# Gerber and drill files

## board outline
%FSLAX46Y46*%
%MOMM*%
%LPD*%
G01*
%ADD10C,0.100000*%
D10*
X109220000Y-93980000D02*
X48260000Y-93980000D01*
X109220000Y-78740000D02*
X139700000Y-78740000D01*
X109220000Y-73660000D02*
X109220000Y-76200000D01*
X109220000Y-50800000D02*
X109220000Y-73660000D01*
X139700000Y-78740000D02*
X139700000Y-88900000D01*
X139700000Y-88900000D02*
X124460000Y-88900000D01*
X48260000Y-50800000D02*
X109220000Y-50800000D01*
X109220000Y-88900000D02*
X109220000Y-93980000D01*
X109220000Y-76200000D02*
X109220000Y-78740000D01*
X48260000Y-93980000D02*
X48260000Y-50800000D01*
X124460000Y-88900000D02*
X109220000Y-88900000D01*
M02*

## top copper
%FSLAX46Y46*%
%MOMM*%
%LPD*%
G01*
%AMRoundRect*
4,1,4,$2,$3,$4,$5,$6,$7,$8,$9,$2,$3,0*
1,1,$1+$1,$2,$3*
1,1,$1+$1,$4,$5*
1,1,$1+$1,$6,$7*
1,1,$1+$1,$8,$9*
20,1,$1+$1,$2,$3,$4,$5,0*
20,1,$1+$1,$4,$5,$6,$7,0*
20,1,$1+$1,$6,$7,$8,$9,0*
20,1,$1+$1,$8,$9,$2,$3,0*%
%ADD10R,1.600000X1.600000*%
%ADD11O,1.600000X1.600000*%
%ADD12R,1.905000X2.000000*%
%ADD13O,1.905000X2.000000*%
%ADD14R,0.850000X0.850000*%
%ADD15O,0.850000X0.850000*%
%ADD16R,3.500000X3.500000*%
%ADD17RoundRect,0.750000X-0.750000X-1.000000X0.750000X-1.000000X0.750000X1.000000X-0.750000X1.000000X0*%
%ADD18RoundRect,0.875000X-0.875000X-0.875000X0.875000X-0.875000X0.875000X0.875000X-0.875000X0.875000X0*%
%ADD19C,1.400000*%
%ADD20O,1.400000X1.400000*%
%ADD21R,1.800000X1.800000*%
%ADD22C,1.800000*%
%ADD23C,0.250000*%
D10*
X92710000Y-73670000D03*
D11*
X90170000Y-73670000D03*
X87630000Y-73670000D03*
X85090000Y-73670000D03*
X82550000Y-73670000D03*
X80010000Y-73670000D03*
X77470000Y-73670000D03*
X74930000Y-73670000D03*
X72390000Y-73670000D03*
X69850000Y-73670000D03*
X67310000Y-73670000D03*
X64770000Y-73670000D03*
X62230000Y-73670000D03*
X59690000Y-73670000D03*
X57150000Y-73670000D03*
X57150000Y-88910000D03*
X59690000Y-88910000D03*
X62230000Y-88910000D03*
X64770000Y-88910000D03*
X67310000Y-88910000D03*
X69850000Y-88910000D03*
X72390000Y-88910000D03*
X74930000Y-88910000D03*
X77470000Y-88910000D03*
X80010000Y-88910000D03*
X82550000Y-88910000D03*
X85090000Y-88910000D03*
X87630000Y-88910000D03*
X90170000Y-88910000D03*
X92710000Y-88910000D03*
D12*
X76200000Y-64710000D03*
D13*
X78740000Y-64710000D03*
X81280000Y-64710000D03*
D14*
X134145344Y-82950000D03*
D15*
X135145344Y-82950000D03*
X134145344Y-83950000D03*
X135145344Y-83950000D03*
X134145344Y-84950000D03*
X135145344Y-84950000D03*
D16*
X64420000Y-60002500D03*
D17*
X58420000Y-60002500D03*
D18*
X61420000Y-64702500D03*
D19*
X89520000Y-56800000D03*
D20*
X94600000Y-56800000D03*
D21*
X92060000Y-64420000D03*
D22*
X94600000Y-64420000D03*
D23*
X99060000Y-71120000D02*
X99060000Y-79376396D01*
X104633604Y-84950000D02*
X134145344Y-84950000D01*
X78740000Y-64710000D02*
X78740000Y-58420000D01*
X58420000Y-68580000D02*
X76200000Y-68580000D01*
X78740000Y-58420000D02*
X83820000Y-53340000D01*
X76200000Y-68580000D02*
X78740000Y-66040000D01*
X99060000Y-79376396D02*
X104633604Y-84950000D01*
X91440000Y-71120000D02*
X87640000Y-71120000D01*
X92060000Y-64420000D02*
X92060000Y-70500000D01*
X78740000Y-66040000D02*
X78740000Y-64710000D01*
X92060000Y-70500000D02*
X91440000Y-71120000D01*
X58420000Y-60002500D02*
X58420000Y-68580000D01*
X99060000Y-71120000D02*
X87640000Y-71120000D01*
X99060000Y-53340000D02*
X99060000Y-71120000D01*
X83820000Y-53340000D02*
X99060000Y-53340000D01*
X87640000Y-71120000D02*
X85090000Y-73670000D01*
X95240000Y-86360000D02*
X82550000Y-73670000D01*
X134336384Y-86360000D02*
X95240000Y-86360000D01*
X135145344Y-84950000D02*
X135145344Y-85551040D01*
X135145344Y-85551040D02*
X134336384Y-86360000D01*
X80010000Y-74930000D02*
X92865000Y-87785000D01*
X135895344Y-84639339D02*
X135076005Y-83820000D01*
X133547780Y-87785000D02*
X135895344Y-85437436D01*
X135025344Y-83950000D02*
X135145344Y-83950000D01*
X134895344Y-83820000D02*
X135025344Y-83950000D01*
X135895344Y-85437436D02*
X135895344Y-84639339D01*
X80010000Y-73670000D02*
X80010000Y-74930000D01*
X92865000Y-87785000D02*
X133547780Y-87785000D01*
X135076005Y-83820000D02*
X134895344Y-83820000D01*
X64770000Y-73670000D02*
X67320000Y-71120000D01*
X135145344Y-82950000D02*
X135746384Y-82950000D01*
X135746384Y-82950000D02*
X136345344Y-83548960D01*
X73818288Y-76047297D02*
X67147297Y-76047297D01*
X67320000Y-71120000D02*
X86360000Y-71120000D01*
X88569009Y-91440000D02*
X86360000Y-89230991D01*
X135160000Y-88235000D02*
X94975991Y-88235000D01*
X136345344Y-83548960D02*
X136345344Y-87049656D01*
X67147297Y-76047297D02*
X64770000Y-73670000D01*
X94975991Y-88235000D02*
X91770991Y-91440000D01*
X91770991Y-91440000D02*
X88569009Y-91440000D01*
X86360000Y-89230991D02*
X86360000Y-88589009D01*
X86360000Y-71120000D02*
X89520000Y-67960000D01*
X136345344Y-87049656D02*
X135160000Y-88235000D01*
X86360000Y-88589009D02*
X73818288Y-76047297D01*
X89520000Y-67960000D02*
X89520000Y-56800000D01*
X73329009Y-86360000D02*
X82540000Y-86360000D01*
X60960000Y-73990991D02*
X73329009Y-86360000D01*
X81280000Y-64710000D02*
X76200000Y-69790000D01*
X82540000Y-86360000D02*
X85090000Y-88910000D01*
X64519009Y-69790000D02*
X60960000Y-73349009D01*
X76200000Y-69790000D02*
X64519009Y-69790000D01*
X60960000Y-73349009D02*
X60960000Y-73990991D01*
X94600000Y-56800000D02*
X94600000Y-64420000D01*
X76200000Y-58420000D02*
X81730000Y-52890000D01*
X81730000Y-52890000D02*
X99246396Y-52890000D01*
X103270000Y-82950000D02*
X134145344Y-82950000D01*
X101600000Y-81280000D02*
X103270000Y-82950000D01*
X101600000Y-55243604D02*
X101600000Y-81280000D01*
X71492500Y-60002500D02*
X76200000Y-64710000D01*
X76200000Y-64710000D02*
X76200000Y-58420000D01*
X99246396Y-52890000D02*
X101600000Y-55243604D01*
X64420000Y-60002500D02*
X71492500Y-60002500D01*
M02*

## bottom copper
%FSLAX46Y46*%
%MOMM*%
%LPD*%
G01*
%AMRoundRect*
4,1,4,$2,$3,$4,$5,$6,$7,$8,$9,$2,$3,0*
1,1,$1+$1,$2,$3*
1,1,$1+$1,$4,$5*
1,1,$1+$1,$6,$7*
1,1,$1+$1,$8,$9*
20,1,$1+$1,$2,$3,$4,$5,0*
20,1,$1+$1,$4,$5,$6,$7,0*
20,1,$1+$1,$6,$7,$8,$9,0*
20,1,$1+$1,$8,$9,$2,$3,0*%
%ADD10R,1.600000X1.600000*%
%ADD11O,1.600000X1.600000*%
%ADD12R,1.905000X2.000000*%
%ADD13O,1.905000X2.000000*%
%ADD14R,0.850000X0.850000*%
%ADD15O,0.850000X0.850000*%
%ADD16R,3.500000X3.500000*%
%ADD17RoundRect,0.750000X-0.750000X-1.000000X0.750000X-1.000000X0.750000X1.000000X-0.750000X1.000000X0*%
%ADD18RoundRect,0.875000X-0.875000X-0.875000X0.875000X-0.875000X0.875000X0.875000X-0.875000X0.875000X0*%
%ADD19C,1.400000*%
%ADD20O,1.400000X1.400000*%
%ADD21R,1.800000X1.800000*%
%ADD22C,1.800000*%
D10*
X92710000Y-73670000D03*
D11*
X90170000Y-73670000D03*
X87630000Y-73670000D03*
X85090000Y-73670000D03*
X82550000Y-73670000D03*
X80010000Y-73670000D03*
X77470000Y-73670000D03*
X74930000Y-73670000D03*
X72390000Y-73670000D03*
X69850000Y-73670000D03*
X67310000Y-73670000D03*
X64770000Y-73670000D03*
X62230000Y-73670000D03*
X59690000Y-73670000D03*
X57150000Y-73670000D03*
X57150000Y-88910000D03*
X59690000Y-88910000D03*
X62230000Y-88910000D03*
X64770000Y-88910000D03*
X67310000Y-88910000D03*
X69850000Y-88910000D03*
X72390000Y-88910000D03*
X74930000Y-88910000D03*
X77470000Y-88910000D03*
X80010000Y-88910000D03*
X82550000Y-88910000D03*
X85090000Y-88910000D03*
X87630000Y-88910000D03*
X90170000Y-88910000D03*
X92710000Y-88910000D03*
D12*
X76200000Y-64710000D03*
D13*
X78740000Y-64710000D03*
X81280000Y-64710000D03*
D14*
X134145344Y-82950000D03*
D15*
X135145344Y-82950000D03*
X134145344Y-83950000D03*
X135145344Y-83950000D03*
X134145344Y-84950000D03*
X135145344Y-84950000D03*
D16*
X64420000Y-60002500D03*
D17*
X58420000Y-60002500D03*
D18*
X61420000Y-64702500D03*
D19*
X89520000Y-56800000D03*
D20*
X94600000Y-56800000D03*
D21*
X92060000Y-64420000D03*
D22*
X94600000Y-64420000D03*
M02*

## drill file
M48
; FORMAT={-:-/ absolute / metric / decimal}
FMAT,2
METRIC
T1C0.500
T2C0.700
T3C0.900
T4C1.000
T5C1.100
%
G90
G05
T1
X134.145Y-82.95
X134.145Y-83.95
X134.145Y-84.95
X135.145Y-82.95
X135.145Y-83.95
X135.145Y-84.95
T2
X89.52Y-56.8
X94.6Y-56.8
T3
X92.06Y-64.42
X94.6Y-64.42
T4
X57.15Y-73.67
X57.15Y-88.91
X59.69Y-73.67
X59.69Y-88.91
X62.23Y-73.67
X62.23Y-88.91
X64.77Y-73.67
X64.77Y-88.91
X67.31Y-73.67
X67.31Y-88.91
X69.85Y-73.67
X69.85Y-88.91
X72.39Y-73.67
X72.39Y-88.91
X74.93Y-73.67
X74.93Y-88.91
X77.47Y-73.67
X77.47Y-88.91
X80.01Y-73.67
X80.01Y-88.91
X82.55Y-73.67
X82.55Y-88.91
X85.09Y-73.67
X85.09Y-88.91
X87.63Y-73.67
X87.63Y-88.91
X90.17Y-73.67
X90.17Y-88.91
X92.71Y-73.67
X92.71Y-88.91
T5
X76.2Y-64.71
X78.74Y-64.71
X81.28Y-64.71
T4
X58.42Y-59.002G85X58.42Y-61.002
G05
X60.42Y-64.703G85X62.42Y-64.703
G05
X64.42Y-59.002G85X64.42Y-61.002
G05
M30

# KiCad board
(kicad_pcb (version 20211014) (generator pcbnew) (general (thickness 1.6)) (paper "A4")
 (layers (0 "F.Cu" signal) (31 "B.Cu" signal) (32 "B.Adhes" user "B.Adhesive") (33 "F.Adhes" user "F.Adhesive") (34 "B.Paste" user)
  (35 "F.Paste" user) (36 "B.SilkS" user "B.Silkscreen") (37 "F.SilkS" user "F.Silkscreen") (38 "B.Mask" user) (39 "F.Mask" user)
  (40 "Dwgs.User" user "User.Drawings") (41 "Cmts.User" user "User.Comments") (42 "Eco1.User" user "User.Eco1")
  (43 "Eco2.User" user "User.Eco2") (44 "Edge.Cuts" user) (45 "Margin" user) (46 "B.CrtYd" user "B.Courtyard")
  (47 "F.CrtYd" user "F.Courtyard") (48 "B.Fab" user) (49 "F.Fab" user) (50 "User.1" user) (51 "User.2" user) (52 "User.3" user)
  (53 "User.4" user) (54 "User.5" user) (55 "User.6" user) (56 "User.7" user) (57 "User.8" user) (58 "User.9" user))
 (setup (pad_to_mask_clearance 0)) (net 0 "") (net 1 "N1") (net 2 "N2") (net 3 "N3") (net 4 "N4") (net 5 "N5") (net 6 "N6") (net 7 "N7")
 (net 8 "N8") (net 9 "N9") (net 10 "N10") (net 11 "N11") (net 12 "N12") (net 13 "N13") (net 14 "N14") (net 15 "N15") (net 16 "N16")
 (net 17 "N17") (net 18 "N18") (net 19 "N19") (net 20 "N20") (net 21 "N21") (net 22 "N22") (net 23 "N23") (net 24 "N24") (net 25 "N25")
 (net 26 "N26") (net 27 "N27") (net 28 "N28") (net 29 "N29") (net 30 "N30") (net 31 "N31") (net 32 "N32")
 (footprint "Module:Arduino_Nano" (layer "F.Cu") (at 92.71 73.67 -90)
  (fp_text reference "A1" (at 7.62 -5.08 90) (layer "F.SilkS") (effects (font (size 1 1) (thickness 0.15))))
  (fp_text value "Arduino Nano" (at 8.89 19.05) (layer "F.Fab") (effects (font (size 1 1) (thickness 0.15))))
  (pad "1" thru_hole rect (at 0 0 270) (size 1.6 1.6) (drill 1) (layers *.Cu *.Mask) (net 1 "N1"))
  (pad "2" thru_hole oval (at 0 2.54 270) (size 1.6 1.6) (drill 1) (layers *.Cu *.Mask) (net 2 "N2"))
  (pad "3" thru_hole oval (at 0 5.08 270) (size 1.6 1.6) (drill 1) (layers *.Cu *.Mask) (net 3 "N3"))
  (pad "4" thru_hole oval (at 0 7.62 270) (size 1.6 1.6) (drill 1) (layers *.Cu *.Mask) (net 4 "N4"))
  (pad "5" thru_hole oval (at 0 10.16 270) (size 1.6 1.6) (drill 1) (layers *.Cu *.Mask) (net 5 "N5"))
  (pad "6" thru_hole oval (at 0 12.7 270) (size 1.6 1.6) (drill 1) (layers *.Cu *.Mask) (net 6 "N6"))
  (pad "7" thru_hole oval (at 0 15.24 270) (size 1.6 1.6) (drill 1) (layers *.Cu *.Mask) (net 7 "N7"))
  (pad "8" thru_hole oval (at 0 17.78 270) (size 1.6 1.6) (drill 1) (layers *.Cu *.Mask) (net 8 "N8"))
  (pad "9" thru_hole oval (at 0 20.32 270) (size 1.6 1.6) (drill 1) (layers *.Cu *.Mask) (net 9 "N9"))
  (pad "10" thru_hole oval (at 0 22.86 270) (size 1.6 1.6) (drill 1) (layers *.Cu *.Mask) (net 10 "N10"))
  (pad "11" thru_hole oval (at 0 25.4 270) (size 1.6 1.6) (drill 1) (layers *.Cu *.Mask) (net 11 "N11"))
  (pad "12" thru_hole oval (at 0 27.94 270) (size 1.6 1.6) (drill 1) (layers *.Cu *.Mask) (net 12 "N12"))
  (pad "13" thru_hole oval (at 0 30.48 270) (size 1.6 1.6) (drill 1) (layers *.Cu *.Mask) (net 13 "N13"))
  (pad "14" thru_hole oval (at 0 33.02 270) (size 1.6 1.6) (drill 1) (layers *.Cu *.Mask) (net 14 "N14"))
  (pad "15" thru_hole oval (at 0 35.56 270) (size 1.6 1.6) (drill 1) (layers *.Cu *.Mask) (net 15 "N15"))
  (pad "16" thru_hole oval (at 15.24 35.56 270) (size 1.6 1.6) (drill 1) (layers *.Cu *.Mask) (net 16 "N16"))
  (pad "17" thru_hole oval (at 15.24 33.02 270) (size 1.6 1.6) (drill 1) (layers *.Cu *.Mask) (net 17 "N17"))
  (pad "18" thru_hole oval (at 15.24 30.48 270) (size 1.6 1.6) (drill 1) (layers *.Cu *.Mask) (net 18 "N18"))
  (pad "19" thru_hole oval (at 15.24 27.94 270) (size 1.6 1.6) (drill 1) (layers *.Cu *.Mask) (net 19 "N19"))
  (pad "20" thru_hole oval (at 15.24 25.4 270) (size 1.6 1.6) (drill 1) (layers *.Cu *.Mask) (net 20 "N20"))
  (pad "21" thru_hole oval (at 15.24 22.86 270) (size 1.6 1.6) (drill 1) (layers *.Cu *.Mask) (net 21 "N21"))
  (pad "22" thru_hole oval (at 15.24 20.32 270) (size 1.6 1.6) (drill 1) (layers *.Cu *.Mask) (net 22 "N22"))
  (pad "23" thru_hole oval (at 15.24 17.78 270) (size 1.6 1.6) (drill 1) (layers *.Cu *.Mask) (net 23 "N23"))
  (pad "24" thru_hole oval (at 15.24 15.24 270) (size 1.6 1.6) (drill 1) (layers *.Cu *.Mask) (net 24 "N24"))
  (pad "25" thru_hole oval (at 15.24 12.7 270) (size 1.6 1.6) (drill 1) (layers *.Cu *.Mask) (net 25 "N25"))
  (pad "26" thru_hole oval (at 15.24 10.16 270) (size 1.6 1.6) (drill 1) (layers *.Cu *.Mask) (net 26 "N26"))
  (pad "27" thru_hole oval (at 15.24 7.62 270) (size 1.6 1.6) (drill 1) (layers *.Cu *.Mask) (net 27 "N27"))
  (pad "28" thru_hole oval (at 15.24 5.08 270) (size 1.6 1.6) (drill 1) (layers *.Cu *.Mask) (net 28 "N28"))
  (pad "29" thru_hole oval (at 15.24 2.54 270) (size 1.6 1.6) (drill 1) (layers *.Cu *.Mask) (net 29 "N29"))
  (pad "30" thru_hole oval (at 15.24 0 270) (size 1.6 1.6) (drill 1) (layers *.Cu *.Mask) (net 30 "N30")))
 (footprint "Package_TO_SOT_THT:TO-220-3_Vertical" (layer "F.Cu") (at 76.2 64.71)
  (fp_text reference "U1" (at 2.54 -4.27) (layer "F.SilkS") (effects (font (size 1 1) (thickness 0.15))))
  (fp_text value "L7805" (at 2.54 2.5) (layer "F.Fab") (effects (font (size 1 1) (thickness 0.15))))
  (pad "1" thru_hole rect (at 0 0) (size 1.905 2) (drill 1.1) (layers *.Cu *.Mask) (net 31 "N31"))
  (pad "2" thru_hole oval (at 2.54 0) (size 1.905 2) (drill 1.1) (layers *.Cu *.Mask) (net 4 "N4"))
  (pad "3" thru_hole oval (at 5.08 0) (size 1.905 2) (drill 1.1) (layers *.Cu *.Mask) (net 27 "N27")))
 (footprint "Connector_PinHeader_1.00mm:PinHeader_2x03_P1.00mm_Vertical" (layer "F.Cu") (at 134.145344 82.95)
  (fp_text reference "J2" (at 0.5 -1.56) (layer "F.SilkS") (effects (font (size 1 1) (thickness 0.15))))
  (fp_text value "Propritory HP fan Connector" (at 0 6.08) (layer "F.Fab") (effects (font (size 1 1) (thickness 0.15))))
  (pad "1" thru_hole rect (at 0 0) (size 0.85 0.85) (drill 0.5) (layers *.Cu *.Mask) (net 31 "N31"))
  (pad "2" thru_hole oval (at 1 0) (size 0.85 0.85) (drill 0.5) (layers *.Cu *.Mask) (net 12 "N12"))
  (pad "3" thru_hole oval (at 0 1) (size 0.85 0.85) (drill 0.5) (layers *.Cu *.Mask) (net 31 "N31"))
  (pad "4" thru_hole oval (at 1 1) (size 0.85 0.85) (drill 0.5) (layers *.Cu *.Mask) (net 6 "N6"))
  (pad "5" thru_hole oval (at 0 2) (size 0.85 0.85) (drill 0.5) (layers *.Cu *.Mask) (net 4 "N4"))
  (pad "6" thru_hole oval (at 1 2) (size 0.85 0.85) (drill 0.5) (layers *.Cu *.Mask) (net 5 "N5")))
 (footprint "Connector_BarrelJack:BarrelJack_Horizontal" (layer "F.Cu") (at 64.42 60.0025)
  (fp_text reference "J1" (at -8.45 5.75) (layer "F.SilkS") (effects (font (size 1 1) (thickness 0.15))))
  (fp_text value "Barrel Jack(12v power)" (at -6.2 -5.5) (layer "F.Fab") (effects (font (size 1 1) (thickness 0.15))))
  (pad "1" thru_hole rect (at 0 0) (size 3.5 3.5) (drill oval 1 3) (layers *.Cu *.Mask) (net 31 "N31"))
  (pad "2" thru_hole roundrect (at -6 0) (size 3 3.5) (drill oval 1 3) (layers *.Cu *.Mask) (roundrect_rratio 0.25) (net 4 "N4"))
  (pad "3" thru_hole roundrect (at -3 4.7) (size 3.5 3.5) (drill oval 3 1) (layers *.Cu *.Mask) (roundrect_rratio 0.25)))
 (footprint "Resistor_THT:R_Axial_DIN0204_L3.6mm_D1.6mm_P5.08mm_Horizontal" (layer "F.Cu") (at 89.52 56.8)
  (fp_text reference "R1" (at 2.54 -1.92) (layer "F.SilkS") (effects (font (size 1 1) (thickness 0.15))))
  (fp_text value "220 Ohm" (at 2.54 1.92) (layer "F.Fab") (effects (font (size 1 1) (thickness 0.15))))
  (pad "1" thru_hole circle (at 0 0) (size 1.4 1.4) (drill 0.7) (layers *.Cu *.Mask) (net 12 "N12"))
  (pad "2" thru_hole oval (at 5.08 0) (size 1.4 1.4) (drill 0.7) (layers *.Cu *.Mask) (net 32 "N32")))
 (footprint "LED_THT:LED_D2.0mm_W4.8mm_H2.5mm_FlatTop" (layer "F.Cu") (at 92.06 64.42)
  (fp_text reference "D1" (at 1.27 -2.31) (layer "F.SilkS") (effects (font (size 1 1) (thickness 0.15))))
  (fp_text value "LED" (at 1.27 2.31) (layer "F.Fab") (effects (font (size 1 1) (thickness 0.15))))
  (pad "1" thru_hole rect (at 0 0) (size 1.8 1.8) (drill 0.9) (layers *.Cu *.Mask) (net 4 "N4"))
  (pad "2" thru_hole circle (at 2.54 0) (size 1.8 1.8) (drill 0.9) (layers *.Cu *.Mask) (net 32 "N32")))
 (gr_line (start 109.22 93.98) (end 48.26 93.98) (layer "Edge.Cuts") (width 0.1))
 (gr_line (start 109.22 78.74) (end 139.7 78.74) (layer "Edge.Cuts") (width 0.1))
 (gr_line (start 109.22 73.66) (end 109.22 76.2) (layer "Edge.Cuts") (width 0.1))
 (gr_line (start 109.22 50.8) (end 109.22 73.66) (layer "Edge.Cuts") (width 0.1))
 (gr_line (start 139.7 78.74) (end 139.7 88.9) (layer "Edge.Cuts") (width 0.1))
 (gr_line (start 139.7 88.9) (end 124.46 88.9) (layer "Edge.Cuts") (width 0.1))
 (gr_line (start 48.26 50.8) (end 109.22 50.8) (layer "Edge.Cuts") (width 0.1))
 (gr_line (start 109.22 88.9) (end 109.22 93.98) (layer "Edge.Cuts") (width 0.1))
 (gr_line (start 109.22 76.2) (end 109.22 78.74) (layer "Edge.Cuts") (width 0.1))
 (gr_line (start 48.26 93.98) (end 48.26 50.8) (layer "Edge.Cuts") (width 0.1))
 (gr_line (start 124.46 88.9) (end 109.22 88.9) (layer "Edge.Cuts") (width 0.1))
 (segment (start 99.06 71.12) (end 99.06 79.376396) (width 0.25) (layer "F.Cu") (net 4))
 (segment (start 104.633604 84.95) (end 134.145344 84.95) (width 0.25) (layer "F.Cu") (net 4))
 (segment (start 78.74 64.71) (end 78.74 58.42) (width 0.25) (layer "F.Cu") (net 4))
 (segment (start 58.42 68.58) (end 76.2 68.58) (width 0.25) (layer "F.Cu") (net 4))
 (segment (start 78.74 58.42) (end 83.82 53.34) (width 0.25) (layer "F.Cu") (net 4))
 (segment (start 76.2 68.58) (end 78.74 66.04) (width 0.25) (layer "F.Cu") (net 4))
 (segment (start 99.06 79.376396) (end 104.633604 84.95) (width 0.25) (layer "F.Cu") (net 4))
 (segment (start 91.44 71.12) (end 87.64 71.12) (width 0.25) (layer "F.Cu") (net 4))
 (segment (start 92.06 64.42) (end 92.06 70.5) (width 0.25) (layer "F.Cu") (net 4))
 (segment (start 78.74 66.04) (end 78.74 64.71) (width 0.25) (layer "F.Cu") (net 4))
 (segment (start 92.06 70.5) (end 91.44 71.12) (width 0.25) (layer "F.Cu") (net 4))
 (segment (start 58.42 60.0025) (end 58.42 68.58) (width 0.25) (layer "F.Cu") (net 4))
 (segment (start 99.06 71.12) (end 87.64 71.12) (width 0.25) (layer "F.Cu") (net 4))
 (segment (start 99.06 53.34) (end 99.06 71.12) (width 0.25) (layer "F.Cu") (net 4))
 (segment (start 83.82 53.34) (end 99.06 53.34) (width 0.25) (layer "F.Cu") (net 4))
 (segment (start 87.64 71.12) (end 85.09 73.67) (width 0.25) (layer "F.Cu") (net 4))
 (segment (start 95.24 86.36) (end 82.55 73.67) (width 0.25) (layer "F.Cu") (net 5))
 (segment (start 134.336384 86.36) (end 95.24 86.36) (width 0.25) (layer "F.Cu") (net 5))
 (segment (start 135.145344 84.95) (end 135.145344 85.55104) (width 0.25) (layer "F.Cu") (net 5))
 (segment (start 135.145344 85.55104) (end 134.336384 86.36) (width 0.25) (layer "F.Cu") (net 5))
 (segment (start 80.01 74.93) (end 92.865 87.785) (width 0.25) (layer "F.Cu") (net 6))
 (segment (start 135.895344 84.639339) (end 135.076005 83.82) (width 0.25) (layer "F.Cu") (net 6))
 (segment (start 133.54778 87.785) (end 135.895344 85.437436) (width 0.25) (layer "F.Cu") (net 6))
 (segment (start 135.025344 83.95) (end 135.145344 83.95) (width 0.25) (layer "F.Cu") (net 6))
 (segment (start 134.895344 83.82) (end 135.025344 83.95) (width 0.25) (layer "F.Cu") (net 6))
 (segment (start 135.895344 85.437436) (end 135.895344 84.639339) (width 0.25) (layer "F.Cu") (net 6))
 (segment (start 80.01 73.67) (end 80.01 74.93) (width 0.25) (layer "F.Cu") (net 6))
 (segment (start 92.865 87.785) (end 133.54778 87.785) (width 0.25) (layer "F.Cu") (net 6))
 (segment (start 135.076005 83.82) (end 134.895344 83.82) (width 0.25) (layer "F.Cu") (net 6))
 (segment (start 64.77 73.67) (end 67.32 71.12) (width 0.25) (layer "F.Cu") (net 12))
 (segment (start 135.145344 82.95) (end 135.746384 82.95) (width 0.25) (layer "F.Cu") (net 12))
 (segment (start 135.746384 82.95) (end 136.345344 83.54896) (width 0.25) (layer "F.Cu") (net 12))
 (segment (start 73.818288 76.047297) (end 67.147297 76.047297) (width 0.25) (layer "F.Cu") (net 12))
 (segment (start 67.32 71.12) (end 86.36 71.12) (width 0.25) (layer "F.Cu") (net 12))
 (segment (start 88.569009 91.44) (end 86.36 89.230991) (width 0.25) (layer "F.Cu") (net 12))
 (segment (start 135.16 88.235) (end 94.975991 88.235) (width 0.25) (layer "F.Cu") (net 12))
 (segment (start 136.345344 83.54896) (end 136.345344 87.049656) (width 0.25) (layer "F.Cu") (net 12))
 (segment (start 67.147297 76.047297) (end 64.77 73.67) (width 0.25) (layer "F.Cu") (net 12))
 (segment (start 94.975991 88.235) (end 91.770991 91.44) (width 0.25) (layer "F.Cu") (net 12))
 (segment (start 91.770991 91.44) (end 88.569009 91.44) (width 0.25) (layer "F.Cu") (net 12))
 (segment (start 86.36 89.230991) (end 86.36 88.589009) (width 0.25) (layer "F.Cu") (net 12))
 (segment (start 86.36 71.12) (end 89.52 67.96) (width 0.25) (layer "F.Cu") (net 12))
 (segment (start 136.345344 87.049656) (end 135.16 88.235) (width 0.25) (layer "F.Cu") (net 12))
 (segment (start 86.36 88.589009) (end 73.818288 76.047297) (width 0.25) (layer "F.Cu") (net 12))
 (segment (start 89.52 67.96) (end 89.52 56.8) (width 0.25) (layer "F.Cu") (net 12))
 (segment (start 73.329009 86.36) (end 82.54 86.36) (width 0.25) (layer "F.Cu") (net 27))
 (segment (start 60.96 73.990991) (end 73.329009 86.36) (width 0.25) (layer "F.Cu") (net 27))
 (segment (start 81.28 64.71) (end 76.2 69.79) (width 0.25) (layer "F.Cu") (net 27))
 (segment (start 82.54 86.36) (end 85.09 88.91) (width 0.25) (layer "F.Cu") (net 27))
 (segment (start 64.519009 69.79) (end 60.96 73.349009) (width 0.25) (layer "F.Cu") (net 27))
 (segment (start 76.2 69.79) (end 64.519009 69.79) (width 0.25) (layer "F.Cu") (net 27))
 (segment (start 60.96 73.349009) (end 60.96 73.990991) (width 0.25) (layer "F.Cu") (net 27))
 (segment (start 94.6 56.8) (end 94.6 64.42) (width 0.25) (layer "F.Cu") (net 32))
 (segment (start 76.2 58.42) (end 81.73 52.89) (width 0.25) (layer "F.Cu") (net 31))
 (segment (start 81.73 52.89) (end 99.246396 52.89) (width 0.25) (layer "F.Cu") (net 31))
 (segment (start 103.27 82.95) (end 134.145344 82.95) (width 0.25) (layer "F.Cu") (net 31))
 (segment (start 101.6 81.28) (end 103.27 82.95) (width 0.25) (layer "F.Cu") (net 31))
 (segment (start 101.6 55.243604) (end 101.6 81.28) (width 0.25) (layer "F.Cu") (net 31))
 (segment (start 71.4925 60.0025) (end 76.2 64.71) (width 0.25) (layer "F.Cu") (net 31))
 (segment (start 76.2 64.71) (end 76.2 58.42) (width 0.25) (layer "F.Cu") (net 31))
 (segment (start 99.246396 52.89) (end 101.6 55.243604) (width 0.25) (layer "F.Cu") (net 31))
 (segment (start 64.42 60.0025) (end 71.4925 60.0025) (width 0.25) (layer "F.Cu") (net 31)))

